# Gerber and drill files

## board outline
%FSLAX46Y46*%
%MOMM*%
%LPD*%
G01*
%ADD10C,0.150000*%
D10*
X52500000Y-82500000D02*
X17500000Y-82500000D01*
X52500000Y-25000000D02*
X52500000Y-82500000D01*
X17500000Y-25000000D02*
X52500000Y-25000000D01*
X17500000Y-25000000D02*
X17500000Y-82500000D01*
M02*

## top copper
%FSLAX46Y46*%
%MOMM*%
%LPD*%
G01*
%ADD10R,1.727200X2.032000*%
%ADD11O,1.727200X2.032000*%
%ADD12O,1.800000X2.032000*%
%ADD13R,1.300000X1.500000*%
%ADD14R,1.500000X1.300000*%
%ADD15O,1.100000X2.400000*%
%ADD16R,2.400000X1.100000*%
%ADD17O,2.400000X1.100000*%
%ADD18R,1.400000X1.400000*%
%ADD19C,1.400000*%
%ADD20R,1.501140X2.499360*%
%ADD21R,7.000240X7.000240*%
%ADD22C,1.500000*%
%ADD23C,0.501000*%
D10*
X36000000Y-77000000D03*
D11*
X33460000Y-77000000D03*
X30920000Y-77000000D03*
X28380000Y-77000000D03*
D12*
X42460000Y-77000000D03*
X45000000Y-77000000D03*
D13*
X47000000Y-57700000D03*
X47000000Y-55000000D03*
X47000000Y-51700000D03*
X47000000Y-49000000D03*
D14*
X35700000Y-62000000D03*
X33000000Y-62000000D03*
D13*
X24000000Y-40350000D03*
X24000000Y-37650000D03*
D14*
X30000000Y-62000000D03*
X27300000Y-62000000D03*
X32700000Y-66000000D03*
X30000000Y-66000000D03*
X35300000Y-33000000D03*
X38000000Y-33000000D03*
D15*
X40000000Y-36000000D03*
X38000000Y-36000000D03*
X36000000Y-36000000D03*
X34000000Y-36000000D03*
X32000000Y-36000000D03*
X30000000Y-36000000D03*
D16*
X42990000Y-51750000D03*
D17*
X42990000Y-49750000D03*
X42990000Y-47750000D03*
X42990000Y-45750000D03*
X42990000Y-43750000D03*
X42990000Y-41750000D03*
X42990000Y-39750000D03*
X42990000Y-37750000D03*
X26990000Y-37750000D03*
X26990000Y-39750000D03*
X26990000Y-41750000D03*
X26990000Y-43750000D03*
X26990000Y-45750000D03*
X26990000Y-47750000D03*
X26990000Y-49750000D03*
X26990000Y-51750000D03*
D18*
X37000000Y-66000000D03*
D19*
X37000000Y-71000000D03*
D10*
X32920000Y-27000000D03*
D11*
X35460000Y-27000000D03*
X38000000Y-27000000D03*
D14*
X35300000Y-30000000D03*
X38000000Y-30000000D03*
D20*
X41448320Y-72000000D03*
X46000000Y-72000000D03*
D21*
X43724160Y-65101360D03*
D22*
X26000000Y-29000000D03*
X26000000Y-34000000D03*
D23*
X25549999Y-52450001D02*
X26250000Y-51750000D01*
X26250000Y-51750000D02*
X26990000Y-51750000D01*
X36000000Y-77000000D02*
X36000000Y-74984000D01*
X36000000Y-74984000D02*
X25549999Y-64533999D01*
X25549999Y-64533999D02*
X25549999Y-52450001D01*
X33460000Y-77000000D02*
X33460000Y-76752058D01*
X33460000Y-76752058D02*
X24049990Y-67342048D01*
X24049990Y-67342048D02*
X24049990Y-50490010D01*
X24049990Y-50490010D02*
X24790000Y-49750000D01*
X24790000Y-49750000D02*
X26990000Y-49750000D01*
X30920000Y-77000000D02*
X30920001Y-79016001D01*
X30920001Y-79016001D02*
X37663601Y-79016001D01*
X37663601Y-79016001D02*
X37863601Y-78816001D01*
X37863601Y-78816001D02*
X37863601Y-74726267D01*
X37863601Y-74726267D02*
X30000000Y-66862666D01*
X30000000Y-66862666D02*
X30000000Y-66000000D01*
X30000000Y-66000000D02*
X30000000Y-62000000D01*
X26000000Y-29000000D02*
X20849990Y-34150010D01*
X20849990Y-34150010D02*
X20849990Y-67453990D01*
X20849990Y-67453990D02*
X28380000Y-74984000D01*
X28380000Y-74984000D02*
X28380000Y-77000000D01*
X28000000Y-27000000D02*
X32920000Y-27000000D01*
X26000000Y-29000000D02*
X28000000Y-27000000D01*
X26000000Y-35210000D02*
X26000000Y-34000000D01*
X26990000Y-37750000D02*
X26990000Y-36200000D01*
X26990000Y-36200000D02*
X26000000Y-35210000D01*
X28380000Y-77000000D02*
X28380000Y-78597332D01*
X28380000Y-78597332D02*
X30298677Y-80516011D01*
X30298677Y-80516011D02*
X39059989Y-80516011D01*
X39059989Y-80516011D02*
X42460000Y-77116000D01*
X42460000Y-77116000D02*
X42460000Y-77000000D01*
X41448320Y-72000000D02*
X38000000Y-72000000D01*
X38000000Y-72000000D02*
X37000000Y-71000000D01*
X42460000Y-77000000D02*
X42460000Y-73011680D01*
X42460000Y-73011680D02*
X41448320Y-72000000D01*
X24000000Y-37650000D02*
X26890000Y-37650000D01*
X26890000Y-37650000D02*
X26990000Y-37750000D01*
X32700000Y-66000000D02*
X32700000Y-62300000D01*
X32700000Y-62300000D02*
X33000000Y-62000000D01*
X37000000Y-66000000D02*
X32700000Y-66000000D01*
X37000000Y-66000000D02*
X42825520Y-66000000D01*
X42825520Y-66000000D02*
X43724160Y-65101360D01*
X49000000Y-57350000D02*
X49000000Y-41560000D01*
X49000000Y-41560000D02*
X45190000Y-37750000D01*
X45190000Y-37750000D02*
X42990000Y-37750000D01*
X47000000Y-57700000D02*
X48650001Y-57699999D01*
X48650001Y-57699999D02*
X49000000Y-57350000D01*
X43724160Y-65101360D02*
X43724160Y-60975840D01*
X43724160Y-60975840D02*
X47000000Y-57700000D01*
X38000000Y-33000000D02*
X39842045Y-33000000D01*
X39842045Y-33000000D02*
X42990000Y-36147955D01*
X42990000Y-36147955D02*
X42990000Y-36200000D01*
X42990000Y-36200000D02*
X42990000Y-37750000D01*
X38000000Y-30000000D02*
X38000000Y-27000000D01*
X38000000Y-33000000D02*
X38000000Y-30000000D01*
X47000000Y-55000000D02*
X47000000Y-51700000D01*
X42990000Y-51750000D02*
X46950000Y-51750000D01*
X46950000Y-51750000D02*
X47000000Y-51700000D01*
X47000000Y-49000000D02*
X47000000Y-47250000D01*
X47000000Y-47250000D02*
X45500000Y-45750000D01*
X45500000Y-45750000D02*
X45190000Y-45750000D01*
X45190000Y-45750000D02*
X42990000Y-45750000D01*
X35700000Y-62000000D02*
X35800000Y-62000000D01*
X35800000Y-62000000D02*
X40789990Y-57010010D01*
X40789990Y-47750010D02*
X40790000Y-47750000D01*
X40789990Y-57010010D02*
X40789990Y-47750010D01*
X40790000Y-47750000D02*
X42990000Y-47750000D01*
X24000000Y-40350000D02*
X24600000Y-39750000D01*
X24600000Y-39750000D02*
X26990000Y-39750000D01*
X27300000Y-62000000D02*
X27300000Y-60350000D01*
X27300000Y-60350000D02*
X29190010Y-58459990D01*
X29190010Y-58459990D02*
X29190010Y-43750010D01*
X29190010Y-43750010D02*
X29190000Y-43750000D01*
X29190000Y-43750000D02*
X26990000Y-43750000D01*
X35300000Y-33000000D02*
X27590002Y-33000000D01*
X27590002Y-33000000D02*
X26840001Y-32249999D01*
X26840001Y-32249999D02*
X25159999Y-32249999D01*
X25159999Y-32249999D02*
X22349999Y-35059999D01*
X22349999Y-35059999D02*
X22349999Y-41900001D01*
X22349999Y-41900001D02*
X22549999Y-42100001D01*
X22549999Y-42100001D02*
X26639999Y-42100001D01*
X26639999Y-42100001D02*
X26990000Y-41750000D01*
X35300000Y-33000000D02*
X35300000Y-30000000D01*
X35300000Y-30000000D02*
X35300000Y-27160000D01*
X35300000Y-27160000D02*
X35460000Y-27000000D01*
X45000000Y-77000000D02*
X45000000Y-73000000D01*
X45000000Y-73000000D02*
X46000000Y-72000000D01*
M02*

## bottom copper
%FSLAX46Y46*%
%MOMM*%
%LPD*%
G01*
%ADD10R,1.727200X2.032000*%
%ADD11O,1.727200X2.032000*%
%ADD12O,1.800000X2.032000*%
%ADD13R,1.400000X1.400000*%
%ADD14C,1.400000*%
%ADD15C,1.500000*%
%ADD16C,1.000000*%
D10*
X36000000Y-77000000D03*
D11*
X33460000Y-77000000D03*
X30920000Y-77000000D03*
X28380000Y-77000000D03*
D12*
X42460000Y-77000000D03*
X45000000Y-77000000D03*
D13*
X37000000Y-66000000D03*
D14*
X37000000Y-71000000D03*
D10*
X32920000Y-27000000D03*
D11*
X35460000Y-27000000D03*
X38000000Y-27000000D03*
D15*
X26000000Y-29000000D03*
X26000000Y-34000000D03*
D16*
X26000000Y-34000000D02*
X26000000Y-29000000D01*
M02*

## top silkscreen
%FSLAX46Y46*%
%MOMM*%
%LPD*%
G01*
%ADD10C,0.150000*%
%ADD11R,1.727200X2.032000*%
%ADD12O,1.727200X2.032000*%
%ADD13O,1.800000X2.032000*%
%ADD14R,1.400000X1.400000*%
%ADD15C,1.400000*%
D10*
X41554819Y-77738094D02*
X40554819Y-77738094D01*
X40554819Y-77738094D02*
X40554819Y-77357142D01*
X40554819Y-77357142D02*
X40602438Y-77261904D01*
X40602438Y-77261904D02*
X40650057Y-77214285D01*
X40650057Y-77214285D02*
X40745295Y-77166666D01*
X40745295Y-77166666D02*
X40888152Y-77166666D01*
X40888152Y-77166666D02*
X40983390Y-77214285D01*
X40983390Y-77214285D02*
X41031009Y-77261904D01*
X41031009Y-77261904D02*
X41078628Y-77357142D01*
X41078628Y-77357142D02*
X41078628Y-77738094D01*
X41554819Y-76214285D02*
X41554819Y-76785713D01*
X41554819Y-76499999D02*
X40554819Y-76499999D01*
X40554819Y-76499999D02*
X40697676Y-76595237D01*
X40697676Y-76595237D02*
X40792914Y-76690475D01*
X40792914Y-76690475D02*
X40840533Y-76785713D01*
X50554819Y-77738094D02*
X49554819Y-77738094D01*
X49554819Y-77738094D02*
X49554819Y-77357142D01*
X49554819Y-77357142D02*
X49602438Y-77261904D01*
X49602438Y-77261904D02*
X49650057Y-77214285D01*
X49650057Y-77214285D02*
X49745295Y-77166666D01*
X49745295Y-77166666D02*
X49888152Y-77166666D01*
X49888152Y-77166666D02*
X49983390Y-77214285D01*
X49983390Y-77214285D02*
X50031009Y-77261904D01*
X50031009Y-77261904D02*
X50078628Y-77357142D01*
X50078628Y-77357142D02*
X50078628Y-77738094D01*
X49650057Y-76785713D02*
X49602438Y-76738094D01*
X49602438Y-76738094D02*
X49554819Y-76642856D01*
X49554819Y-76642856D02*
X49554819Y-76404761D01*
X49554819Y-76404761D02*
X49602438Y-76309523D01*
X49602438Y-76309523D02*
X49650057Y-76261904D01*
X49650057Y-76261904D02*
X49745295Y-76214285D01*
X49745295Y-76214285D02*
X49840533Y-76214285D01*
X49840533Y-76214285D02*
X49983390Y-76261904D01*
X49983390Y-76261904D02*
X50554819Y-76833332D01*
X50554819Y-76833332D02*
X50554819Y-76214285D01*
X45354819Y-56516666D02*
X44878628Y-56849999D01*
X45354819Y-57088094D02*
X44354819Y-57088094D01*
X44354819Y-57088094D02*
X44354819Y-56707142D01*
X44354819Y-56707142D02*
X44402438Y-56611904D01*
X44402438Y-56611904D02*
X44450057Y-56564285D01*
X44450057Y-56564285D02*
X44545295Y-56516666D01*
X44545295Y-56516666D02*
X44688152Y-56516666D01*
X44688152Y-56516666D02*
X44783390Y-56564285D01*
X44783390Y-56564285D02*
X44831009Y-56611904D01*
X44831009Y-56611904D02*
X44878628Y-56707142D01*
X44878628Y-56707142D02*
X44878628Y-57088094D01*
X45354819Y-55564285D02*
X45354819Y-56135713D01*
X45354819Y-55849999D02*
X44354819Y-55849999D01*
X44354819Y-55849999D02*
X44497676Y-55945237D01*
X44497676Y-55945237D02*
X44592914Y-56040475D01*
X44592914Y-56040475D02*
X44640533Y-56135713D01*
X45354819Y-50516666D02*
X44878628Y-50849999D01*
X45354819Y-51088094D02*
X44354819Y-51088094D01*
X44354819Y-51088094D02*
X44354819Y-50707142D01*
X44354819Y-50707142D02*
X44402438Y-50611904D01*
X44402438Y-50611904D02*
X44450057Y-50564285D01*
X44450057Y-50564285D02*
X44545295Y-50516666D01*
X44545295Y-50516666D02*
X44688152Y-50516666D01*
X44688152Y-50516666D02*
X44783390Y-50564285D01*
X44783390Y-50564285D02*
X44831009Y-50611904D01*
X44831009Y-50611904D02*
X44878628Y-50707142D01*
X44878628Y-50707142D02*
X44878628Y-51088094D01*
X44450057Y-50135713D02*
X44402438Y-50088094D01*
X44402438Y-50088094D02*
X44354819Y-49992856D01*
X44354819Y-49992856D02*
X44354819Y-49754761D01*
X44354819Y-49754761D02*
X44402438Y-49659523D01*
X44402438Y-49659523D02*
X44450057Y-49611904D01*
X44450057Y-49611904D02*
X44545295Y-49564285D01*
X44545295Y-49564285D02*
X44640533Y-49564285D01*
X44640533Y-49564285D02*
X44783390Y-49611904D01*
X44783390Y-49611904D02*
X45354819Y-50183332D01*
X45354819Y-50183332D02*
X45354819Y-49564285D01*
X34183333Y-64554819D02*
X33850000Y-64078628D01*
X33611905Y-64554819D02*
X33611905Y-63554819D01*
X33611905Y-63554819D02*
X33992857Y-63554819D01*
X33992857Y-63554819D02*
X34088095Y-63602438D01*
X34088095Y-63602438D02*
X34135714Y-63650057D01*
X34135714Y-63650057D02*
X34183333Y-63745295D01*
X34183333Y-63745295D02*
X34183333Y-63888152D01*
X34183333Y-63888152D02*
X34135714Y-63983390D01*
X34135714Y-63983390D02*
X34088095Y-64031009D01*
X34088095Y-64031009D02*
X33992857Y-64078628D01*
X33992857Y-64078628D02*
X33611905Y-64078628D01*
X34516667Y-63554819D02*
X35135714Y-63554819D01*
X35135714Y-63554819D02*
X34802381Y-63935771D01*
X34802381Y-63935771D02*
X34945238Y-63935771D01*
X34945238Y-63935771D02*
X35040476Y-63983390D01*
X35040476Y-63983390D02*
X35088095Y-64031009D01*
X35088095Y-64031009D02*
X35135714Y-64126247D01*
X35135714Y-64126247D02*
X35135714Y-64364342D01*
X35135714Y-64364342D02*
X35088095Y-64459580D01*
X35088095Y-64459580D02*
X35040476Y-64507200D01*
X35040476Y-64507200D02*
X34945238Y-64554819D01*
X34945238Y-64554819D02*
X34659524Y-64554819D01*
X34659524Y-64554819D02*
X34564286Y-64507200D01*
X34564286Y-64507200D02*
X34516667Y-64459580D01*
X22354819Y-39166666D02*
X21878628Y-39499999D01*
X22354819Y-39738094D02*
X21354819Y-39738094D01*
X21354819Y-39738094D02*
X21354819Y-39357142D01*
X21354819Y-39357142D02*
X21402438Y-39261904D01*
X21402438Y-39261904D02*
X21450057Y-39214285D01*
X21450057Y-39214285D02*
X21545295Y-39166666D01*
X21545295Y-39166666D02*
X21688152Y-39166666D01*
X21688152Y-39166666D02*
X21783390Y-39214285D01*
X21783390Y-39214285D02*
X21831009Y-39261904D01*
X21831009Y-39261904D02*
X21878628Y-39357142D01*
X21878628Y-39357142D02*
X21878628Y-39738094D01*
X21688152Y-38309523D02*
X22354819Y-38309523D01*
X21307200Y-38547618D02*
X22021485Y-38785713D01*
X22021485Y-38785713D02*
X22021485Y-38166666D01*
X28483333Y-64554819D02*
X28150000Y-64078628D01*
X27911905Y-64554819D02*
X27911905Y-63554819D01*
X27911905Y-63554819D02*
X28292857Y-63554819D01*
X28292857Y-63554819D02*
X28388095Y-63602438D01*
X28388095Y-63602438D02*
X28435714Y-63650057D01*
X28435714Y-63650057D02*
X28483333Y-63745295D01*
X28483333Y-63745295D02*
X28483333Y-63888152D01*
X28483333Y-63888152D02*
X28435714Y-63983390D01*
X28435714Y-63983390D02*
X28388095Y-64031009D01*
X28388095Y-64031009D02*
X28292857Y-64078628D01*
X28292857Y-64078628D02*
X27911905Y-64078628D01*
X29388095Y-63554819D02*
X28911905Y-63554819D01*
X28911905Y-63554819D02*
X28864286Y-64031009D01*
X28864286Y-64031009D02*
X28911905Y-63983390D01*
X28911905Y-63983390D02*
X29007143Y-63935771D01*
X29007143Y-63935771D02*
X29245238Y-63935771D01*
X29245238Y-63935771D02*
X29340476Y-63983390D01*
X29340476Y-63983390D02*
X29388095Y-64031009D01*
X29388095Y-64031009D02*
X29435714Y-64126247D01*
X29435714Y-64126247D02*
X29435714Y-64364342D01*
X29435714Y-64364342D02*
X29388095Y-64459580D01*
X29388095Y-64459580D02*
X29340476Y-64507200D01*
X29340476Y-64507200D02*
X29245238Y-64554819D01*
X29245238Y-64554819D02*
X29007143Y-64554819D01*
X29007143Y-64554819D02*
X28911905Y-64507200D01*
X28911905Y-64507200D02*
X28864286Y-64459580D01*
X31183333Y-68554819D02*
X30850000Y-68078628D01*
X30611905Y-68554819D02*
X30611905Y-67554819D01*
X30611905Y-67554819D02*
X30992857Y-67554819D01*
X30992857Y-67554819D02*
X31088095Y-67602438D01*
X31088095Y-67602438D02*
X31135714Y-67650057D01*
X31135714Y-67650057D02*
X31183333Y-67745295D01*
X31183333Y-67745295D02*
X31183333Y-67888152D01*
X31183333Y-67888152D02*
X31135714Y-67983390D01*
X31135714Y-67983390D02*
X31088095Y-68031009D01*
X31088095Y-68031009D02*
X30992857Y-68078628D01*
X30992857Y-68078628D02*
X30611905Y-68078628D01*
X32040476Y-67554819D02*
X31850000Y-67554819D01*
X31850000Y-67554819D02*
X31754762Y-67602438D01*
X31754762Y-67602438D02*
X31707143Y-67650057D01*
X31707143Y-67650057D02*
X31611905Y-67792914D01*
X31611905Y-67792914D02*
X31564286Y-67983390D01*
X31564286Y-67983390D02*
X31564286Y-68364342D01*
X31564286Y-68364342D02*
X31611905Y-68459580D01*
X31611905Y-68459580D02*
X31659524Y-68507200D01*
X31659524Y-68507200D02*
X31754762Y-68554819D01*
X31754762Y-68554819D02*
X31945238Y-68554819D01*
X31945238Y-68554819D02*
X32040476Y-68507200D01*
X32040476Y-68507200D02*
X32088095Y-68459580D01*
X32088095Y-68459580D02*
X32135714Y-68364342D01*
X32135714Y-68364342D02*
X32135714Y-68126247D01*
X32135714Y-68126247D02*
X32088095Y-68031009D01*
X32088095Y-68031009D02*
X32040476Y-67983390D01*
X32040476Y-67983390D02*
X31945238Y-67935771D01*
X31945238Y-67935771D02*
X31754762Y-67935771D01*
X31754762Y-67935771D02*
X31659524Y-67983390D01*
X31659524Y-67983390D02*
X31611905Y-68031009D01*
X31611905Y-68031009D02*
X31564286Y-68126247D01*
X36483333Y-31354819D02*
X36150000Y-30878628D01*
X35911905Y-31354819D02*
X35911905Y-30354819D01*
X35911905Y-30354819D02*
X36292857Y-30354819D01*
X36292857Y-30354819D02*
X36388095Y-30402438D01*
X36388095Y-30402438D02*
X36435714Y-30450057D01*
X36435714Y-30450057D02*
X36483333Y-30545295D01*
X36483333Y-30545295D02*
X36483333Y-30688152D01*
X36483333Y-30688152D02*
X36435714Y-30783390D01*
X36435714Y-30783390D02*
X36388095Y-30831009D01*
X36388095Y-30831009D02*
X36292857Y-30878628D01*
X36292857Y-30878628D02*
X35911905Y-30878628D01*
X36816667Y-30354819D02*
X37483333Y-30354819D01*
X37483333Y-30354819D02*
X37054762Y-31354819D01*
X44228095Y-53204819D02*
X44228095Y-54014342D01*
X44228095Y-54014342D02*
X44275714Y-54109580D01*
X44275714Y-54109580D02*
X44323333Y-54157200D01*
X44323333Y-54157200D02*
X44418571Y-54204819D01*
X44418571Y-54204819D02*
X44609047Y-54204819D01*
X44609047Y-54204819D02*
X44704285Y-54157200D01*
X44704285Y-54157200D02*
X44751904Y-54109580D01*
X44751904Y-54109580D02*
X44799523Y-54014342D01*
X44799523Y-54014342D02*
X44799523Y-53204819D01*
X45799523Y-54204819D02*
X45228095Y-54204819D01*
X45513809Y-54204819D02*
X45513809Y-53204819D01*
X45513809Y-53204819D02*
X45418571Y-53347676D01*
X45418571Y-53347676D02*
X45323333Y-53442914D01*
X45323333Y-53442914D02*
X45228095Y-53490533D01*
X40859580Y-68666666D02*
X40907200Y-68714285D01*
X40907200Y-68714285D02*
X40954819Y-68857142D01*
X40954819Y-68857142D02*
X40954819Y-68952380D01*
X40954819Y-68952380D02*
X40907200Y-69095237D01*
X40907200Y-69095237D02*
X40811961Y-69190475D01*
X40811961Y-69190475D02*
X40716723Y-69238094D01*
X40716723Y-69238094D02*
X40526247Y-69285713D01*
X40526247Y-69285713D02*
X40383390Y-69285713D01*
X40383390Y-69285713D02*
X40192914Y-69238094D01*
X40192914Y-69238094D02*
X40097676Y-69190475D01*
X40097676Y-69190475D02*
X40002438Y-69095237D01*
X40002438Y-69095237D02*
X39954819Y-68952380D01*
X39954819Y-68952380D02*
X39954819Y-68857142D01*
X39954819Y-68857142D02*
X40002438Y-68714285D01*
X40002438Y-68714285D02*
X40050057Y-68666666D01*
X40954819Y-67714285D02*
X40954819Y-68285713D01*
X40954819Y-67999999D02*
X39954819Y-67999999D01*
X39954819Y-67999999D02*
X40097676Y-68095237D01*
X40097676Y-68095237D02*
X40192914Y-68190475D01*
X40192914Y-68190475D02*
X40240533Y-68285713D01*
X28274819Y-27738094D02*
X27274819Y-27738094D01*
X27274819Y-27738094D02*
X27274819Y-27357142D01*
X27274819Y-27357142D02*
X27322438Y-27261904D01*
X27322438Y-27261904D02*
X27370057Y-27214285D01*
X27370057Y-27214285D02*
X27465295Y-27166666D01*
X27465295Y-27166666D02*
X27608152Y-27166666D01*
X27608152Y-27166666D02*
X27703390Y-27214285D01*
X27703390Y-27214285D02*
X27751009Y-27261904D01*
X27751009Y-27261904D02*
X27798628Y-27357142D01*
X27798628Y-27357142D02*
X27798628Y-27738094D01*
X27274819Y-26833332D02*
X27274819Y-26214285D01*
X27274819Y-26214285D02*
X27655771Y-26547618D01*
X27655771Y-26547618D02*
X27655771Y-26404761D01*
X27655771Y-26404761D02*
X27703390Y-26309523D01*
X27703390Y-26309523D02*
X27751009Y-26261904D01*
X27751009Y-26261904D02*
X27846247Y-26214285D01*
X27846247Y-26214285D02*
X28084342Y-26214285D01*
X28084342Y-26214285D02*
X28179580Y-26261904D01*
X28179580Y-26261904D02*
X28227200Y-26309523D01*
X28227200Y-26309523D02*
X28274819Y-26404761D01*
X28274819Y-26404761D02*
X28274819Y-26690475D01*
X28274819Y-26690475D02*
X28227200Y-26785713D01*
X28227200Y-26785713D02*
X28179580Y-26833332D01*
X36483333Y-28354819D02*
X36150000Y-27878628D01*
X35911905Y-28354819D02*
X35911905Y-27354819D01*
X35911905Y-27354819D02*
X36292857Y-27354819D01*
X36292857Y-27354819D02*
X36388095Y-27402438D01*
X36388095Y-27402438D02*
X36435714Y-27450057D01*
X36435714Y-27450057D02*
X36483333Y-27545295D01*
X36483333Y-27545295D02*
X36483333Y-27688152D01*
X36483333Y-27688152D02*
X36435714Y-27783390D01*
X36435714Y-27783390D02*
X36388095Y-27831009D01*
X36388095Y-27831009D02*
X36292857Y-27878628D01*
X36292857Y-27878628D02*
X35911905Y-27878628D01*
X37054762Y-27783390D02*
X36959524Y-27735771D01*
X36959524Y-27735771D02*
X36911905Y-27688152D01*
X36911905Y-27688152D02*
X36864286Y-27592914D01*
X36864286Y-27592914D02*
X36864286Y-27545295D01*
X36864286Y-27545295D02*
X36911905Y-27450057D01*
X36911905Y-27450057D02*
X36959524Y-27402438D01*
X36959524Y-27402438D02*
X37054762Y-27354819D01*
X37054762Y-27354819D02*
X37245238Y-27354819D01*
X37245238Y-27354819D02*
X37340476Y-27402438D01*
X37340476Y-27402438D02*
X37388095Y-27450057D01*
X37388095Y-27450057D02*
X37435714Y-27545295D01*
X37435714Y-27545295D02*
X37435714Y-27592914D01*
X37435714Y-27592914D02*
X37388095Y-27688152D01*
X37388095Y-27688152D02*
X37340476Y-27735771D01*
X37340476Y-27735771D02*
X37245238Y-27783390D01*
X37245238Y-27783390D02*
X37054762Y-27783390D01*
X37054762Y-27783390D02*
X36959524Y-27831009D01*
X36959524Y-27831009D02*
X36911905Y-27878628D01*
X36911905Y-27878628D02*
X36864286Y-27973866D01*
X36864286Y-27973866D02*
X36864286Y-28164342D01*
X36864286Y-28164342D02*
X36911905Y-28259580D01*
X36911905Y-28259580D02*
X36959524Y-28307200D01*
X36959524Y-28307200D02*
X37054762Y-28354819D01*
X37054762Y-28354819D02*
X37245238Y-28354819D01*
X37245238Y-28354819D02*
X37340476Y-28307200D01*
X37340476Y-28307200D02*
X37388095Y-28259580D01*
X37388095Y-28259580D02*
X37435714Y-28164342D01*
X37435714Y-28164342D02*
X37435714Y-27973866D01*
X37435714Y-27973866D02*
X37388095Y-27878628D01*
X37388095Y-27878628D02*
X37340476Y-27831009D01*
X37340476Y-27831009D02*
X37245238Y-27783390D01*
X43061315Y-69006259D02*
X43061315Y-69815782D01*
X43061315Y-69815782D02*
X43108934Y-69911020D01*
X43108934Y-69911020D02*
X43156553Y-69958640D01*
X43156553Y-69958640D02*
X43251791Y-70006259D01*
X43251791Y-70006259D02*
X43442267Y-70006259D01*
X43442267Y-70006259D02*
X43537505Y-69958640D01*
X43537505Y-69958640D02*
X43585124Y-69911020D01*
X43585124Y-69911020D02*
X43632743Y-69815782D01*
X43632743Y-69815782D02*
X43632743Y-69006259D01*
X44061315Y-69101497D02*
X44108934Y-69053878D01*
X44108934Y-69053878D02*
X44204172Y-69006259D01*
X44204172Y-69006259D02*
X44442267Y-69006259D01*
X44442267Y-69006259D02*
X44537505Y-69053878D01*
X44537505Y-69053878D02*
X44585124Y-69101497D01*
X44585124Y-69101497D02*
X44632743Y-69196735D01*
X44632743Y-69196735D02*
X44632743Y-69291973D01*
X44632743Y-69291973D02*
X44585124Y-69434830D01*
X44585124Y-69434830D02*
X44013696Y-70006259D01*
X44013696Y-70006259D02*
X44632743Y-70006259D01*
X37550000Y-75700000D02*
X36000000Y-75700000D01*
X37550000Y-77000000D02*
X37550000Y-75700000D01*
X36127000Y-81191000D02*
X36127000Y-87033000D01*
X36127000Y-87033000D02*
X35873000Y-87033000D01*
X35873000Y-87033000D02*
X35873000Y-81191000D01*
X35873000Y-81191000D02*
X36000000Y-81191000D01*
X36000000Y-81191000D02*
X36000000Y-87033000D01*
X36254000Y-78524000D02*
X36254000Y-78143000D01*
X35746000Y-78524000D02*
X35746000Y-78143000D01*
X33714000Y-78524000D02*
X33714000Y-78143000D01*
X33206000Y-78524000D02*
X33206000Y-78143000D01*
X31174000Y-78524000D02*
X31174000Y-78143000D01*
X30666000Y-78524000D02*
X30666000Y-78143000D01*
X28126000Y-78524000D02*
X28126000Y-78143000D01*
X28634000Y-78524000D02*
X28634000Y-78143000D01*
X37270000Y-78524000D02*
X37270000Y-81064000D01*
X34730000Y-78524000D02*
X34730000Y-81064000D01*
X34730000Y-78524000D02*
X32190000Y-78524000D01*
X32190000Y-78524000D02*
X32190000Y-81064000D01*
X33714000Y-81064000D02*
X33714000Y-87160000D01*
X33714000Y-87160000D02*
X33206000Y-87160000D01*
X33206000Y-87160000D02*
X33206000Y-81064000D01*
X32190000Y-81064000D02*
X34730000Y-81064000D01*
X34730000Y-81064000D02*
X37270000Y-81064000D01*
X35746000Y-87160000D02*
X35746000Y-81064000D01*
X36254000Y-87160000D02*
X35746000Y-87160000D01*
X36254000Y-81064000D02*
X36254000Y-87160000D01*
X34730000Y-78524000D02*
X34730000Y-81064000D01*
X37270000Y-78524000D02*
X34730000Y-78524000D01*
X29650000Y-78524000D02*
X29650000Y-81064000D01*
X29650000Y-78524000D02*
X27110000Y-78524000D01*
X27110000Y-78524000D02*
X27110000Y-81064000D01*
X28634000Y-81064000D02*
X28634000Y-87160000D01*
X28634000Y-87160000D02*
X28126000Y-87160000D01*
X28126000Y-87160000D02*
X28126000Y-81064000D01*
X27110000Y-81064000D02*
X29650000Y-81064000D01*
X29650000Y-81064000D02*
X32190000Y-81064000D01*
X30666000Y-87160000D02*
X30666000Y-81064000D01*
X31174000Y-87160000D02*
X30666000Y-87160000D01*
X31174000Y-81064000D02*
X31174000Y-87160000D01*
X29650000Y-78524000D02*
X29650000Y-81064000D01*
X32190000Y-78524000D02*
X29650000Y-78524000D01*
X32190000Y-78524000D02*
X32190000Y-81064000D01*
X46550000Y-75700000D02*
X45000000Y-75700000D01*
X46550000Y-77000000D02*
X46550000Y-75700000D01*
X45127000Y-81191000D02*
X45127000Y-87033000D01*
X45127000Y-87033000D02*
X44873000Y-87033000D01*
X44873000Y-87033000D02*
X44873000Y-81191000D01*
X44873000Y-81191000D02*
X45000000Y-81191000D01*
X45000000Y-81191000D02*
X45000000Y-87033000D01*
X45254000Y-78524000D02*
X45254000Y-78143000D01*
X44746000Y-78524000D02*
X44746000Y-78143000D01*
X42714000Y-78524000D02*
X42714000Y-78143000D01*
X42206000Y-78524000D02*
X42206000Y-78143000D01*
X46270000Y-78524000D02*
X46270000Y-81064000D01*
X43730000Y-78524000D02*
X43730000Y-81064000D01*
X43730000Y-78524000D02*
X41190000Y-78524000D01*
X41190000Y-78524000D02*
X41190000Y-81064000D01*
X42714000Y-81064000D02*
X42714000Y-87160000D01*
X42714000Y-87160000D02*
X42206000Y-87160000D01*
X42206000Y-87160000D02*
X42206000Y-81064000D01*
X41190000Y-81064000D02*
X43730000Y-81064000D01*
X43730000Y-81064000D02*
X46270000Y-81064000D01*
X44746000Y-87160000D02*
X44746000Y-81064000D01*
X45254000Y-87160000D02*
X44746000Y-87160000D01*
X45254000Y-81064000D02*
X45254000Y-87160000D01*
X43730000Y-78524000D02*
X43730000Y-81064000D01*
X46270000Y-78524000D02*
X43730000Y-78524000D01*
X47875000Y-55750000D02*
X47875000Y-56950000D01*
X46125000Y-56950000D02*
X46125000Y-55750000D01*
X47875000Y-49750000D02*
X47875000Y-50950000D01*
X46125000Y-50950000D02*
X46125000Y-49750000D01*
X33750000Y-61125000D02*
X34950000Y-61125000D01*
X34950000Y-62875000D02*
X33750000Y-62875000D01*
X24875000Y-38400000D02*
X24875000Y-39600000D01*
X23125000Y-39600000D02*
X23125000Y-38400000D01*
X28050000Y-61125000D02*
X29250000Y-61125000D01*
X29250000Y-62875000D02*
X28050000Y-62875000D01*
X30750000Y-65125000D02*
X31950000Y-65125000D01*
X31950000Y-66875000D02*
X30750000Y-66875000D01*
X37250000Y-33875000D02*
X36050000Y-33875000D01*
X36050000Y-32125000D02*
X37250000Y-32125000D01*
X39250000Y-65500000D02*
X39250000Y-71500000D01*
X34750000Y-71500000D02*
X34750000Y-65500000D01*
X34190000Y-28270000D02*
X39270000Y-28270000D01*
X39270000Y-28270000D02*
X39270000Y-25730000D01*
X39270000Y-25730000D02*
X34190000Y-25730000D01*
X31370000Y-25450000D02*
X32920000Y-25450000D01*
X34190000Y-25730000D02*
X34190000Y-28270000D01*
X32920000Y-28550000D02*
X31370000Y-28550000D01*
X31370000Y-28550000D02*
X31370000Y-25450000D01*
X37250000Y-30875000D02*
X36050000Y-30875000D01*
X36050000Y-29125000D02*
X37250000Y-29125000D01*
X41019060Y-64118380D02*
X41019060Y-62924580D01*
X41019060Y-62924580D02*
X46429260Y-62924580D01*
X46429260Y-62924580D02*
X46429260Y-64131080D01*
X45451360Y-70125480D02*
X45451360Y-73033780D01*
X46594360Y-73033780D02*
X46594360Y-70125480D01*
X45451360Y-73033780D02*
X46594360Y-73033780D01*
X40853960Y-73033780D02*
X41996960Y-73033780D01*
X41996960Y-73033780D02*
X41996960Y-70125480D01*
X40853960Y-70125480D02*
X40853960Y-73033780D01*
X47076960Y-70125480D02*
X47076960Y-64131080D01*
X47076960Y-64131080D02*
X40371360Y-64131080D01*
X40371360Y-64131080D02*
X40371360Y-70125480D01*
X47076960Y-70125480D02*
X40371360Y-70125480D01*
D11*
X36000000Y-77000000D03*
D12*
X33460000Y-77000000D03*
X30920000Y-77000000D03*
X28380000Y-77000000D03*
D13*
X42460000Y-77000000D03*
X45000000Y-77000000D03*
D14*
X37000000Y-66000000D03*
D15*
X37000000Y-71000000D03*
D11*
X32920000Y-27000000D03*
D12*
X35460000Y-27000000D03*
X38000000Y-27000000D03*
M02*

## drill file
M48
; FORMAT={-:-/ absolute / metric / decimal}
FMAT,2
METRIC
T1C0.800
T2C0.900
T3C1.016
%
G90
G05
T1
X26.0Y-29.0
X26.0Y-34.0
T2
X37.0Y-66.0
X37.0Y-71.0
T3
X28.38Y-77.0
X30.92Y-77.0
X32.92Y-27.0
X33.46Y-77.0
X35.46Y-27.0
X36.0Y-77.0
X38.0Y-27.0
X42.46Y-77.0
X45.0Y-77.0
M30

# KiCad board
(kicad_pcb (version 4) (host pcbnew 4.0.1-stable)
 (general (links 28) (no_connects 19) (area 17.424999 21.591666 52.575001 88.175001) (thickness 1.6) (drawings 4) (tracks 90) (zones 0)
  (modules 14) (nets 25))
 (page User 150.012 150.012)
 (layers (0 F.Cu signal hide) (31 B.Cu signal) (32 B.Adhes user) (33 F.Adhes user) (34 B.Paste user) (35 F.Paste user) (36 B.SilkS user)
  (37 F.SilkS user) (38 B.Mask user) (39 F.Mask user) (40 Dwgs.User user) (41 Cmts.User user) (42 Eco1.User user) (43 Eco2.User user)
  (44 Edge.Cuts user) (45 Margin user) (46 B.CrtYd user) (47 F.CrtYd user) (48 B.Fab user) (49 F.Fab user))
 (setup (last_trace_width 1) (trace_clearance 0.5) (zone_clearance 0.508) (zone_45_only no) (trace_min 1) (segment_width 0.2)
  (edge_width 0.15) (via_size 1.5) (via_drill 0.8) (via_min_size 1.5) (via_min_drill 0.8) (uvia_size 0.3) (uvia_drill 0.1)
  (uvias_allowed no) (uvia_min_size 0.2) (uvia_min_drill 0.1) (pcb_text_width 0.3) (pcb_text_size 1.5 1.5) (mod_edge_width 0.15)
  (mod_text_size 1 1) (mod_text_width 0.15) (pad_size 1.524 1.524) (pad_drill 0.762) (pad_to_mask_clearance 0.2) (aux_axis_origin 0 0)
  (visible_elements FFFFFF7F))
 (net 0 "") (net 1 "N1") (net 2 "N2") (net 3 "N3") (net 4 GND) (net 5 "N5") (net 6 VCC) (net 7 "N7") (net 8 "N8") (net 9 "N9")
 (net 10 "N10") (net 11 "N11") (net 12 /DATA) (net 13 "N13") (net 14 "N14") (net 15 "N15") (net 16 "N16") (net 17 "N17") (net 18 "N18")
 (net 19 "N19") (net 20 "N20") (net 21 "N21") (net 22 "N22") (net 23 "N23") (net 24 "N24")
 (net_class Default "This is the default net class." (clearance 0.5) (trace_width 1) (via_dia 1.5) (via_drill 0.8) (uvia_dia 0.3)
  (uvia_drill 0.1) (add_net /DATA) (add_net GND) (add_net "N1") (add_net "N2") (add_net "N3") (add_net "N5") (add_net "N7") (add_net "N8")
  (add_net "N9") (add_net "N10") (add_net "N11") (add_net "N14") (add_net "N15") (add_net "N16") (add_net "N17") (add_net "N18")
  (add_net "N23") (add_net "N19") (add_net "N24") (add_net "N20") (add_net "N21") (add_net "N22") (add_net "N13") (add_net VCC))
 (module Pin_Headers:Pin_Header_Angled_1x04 (layer F.Cu) (at 36 77 270)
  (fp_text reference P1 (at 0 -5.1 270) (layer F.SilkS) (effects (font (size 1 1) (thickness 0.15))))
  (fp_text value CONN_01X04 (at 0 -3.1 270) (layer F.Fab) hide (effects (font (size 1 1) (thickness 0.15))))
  (fp_line (start -1.3 -1.55) (end -1.3 0) (layer F.SilkS) (width 0.15))
  (fp_line (start 0 -1.55) (end -1.3 -1.55) (layer F.SilkS) (width 0.15))
  (fp_line (start 4.191 -0.127) (end 10.033 -0.127) (layer F.SilkS) (width 0.15))
  (fp_line (start 10.033 -0.127) (end 10.033 0.127) (layer F.SilkS) (width 0.15))
  (fp_line (start 10.033 0.127) (end 4.191 0.127) (layer F.SilkS) (width 0.15))
  (fp_line (start 4.191 0.127) (end 4.191 0) (layer F.SilkS) (width 0.15))
  (fp_line (start 4.191 0) (end 10.033 0) (layer F.SilkS) (width 0.15))
  (fp_line (start 1.524 -0.254) (end 1.143 -0.254) (layer F.SilkS) (width 0.15))
  (fp_line (start 1.524 0.254) (end 1.143 0.254) (layer F.SilkS) (width 0.15))
  (fp_line (start 1.524 2.286) (end 1.143 2.286) (layer F.SilkS) (width 0.15))
  (fp_line (start 1.524 2.794) (end 1.143 2.794) (layer F.SilkS) (width 0.15))
  (fp_line (start 1.524 4.826) (end 1.143 4.826) (layer F.SilkS) (width 0.15))
  (fp_line (start 1.524 5.334) (end 1.143 5.334) (layer F.SilkS) (width 0.15))
  (fp_line (start 1.524 7.874) (end 1.143 7.874) (layer F.SilkS) (width 0.15))
  (fp_line (start 1.524 7.366) (end 1.143 7.366) (layer F.SilkS) (width 0.15))
  (fp_line (start 1.524 -1.27) (end 4.064 -1.27) (layer F.SilkS) (width 0.15))
  (fp_line (start 1.524 1.27) (end 4.064 1.27) (layer F.SilkS) (width 0.15))
  (fp_line (start 1.524 1.27) (end 1.524 3.81) (layer F.SilkS) (width 0.15))
  (fp_line (start 1.524 3.81) (end 4.064 3.81) (layer F.SilkS) (width 0.15))
  (fp_line (start 4.064 2.286) (end 10.16 2.286) (layer F.SilkS) (width 0.15))
  (fp_line (start 10.16 2.286) (end 10.16 2.794) (layer F.SilkS) (width 0.15))
  (fp_line (start 10.16 2.794) (end 4.064 2.794) (layer F.SilkS) (width 0.15))
  (fp_line (start 4.064 3.81) (end 4.064 1.27) (layer F.SilkS) (width 0.15))
  (fp_line (start 4.064 1.27) (end 4.064 -1.27) (layer F.SilkS) (width 0.15))
  (fp_line (start 10.16 0.254) (end 4.064 0.254) (layer F.SilkS) (width 0.15))
  (fp_line (start 10.16 -0.254) (end 10.16 0.254) (layer F.SilkS) (width 0.15))
  (fp_line (start 4.064 -0.254) (end 10.16 -0.254) (layer F.SilkS) (width 0.15))
  (fp_line (start 1.524 1.27) (end 4.064 1.27) (layer F.SilkS) (width 0.15))
  (fp_line (start 1.524 -1.27) (end 1.524 1.27) (layer F.SilkS) (width 0.15))
  (fp_line (start 1.524 6.35) (end 4.064 6.35) (layer F.SilkS) (width 0.15))
  (fp_line (start 1.524 6.35) (end 1.524 8.89) (layer F.SilkS) (width 0.15))
  (fp_line (start 1.524 8.89) (end 4.064 8.89) (layer F.SilkS) (width 0.15))
  (fp_line (start 4.064 7.366) (end 10.16 7.366) (layer F.SilkS) (width 0.15))
  (fp_line (start 10.16 7.366) (end 10.16 7.874) (layer F.SilkS) (width 0.15))
  (fp_line (start 10.16 7.874) (end 4.064 7.874) (layer F.SilkS) (width 0.15))
  (fp_line (start 4.064 8.89) (end 4.064 6.35) (layer F.SilkS) (width 0.15))
  (fp_line (start 4.064 6.35) (end 4.064 3.81) (layer F.SilkS) (width 0.15))
  (fp_line (start 10.16 5.334) (end 4.064 5.334) (layer F.SilkS) (width 0.15))
  (fp_line (start 10.16 4.826) (end 10.16 5.334) (layer F.SilkS) (width 0.15))
  (fp_line (start 4.064 4.826) (end 10.16 4.826) (layer F.SilkS) (width 0.15))
  (fp_line (start 1.524 6.35) (end 4.064 6.35) (layer F.SilkS) (width 0.15))
  (fp_line (start 1.524 3.81) (end 1.524 6.35) (layer F.SilkS) (width 0.15))
  (fp_line (start 1.524 3.81) (end 4.064 3.81) (layer F.SilkS) (width 0.15))
  (pad 1 thru_hole rect (at 0 0 270) (size 2.032 1.7272) (drill 1.016) (layers *.Cu *.Mask F.SilkS) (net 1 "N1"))
  (pad 2 thru_hole oval (at 0 2.54 270) (size 2.032 1.7272) (drill 1.016) (layers *.Cu *.Mask F.SilkS) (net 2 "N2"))
  (pad 3 thru_hole oval (at 0 5.08 270) (size 2.032 1.7272) (drill 1.016) (layers *.Cu *.Mask F.SilkS) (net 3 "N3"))
  (pad 4 thru_hole oval (at 0 7.62 270) (size 2.032 1.7272) (drill 1.016) (layers *.Cu *.Mask F.SilkS) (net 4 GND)))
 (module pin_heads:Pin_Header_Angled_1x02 (layer F.Cu) (at 45 77 270)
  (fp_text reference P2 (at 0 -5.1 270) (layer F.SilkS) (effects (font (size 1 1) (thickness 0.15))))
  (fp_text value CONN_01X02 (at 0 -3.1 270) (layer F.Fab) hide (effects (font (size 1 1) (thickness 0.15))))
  (fp_line (start -1.3 -1.55) (end -1.3 0) (layer F.SilkS) (width 0.15))
  (fp_line (start 0 -1.55) (end -1.3 -1.55) (layer F.SilkS) (width 0.15))
  (fp_line (start 4.191 -0.127) (end 10.033 -0.127) (layer F.SilkS) (width 0.15))
  (fp_line (start 10.033 -0.127) (end 10.033 0.127) (layer F.SilkS) (width 0.15))
  (fp_line (start 10.033 0.127) (end 4.191 0.127) (layer F.SilkS) (width 0.15))
  (fp_line (start 4.191 0.127) (end 4.191 0) (layer F.SilkS) (width 0.15))
  (fp_line (start 4.191 0) (end 10.033 0) (layer F.SilkS) (width 0.15))
  (fp_line (start 1.524 -0.254) (end 1.143 -0.254) (layer F.SilkS) (width 0.15))
  (fp_line (start 1.524 0.254) (end 1.143 0.254) (layer F.SilkS) (width 0.15))
  (fp_line (start 1.524 2.286) (end 1.143 2.286) (layer F.SilkS) (width 0.15))
  (fp_line (start 1.524 2.794) (end 1.143 2.794) (layer F.SilkS) (width 0.15))
  (fp_line (start 1.524 -1.27) (end 4.064 -1.27) (layer F.SilkS) (width 0.15))
  (fp_line (start 1.524 1.27) (end 4.064 1.27) (layer F.SilkS) (width 0.15))
  (fp_line (start 1.524 1.27) (end 1.524 3.81) (layer F.SilkS) (width 0.15))
  (fp_line (start 1.524 3.81) (end 4.064 3.81) (layer F.SilkS) (width 0.15))
  (fp_line (start 4.064 2.286) (end 10.16 2.286) (layer F.SilkS) (width 0.15))
  (fp_line (start 10.16 2.286) (end 10.16 2.794) (layer F.SilkS) (width 0.15))
  (fp_line (start 10.16 2.794) (end 4.064 2.794) (layer F.SilkS) (width 0.15))
  (fp_line (start 4.064 3.81) (end 4.064 1.27) (layer F.SilkS) (width 0.15))
  (fp_line (start 4.064 1.27) (end 4.064 -1.27) (layer F.SilkS) (width 0.15))
  (fp_line (start 10.16 0.254) (end 4.064 0.254) (layer F.SilkS) (width 0.15))
  (fp_line (start 10.16 -0.254) (end 10.16 0.254) (layer F.SilkS) (width 0.15))
  (fp_line (start 4.064 -0.254) (end 10.16 -0.254) (layer F.SilkS) (width 0.15))
  (fp_line (start 1.524 1.27) (end 4.064 1.27) (layer F.SilkS) (width 0.15))
  (fp_line (start 1.524 -1.27) (end 1.524 1.27) (layer F.SilkS) (width 0.15))
  (pad 2 thru_hole oval (at 0 2.54 270) (size 2.032 1.8) (drill 1.016) (layers *.Cu *.Mask F.SilkS) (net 4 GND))
  (pad 1 thru_hole oval (at 0 0 270) (size 2.032 1.8) (drill 1.016) (layers *.Cu *.Mask F.SilkS) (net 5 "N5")))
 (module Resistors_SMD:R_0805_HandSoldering (layer F.Cu) (at 47 56.35 90)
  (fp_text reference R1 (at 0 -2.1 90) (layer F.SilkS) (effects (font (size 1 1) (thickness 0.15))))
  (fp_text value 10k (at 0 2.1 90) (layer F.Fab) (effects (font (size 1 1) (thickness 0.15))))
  (fp_line (start 0.6 0.875) (end -0.6 0.875) (layer F.SilkS) (width 0.15))
  (fp_line (start -0.6 -0.875) (end 0.6 -0.875) (layer F.SilkS) (width 0.15))
  (pad 1 smd rect (at -1.35 0 90) (size 1.5 1.3) (layers F.Cu F.Paste F.Mask) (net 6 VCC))
  (pad 2 smd rect (at 1.35 0 90) (size 1.5 1.3) (layers F.Cu F.Paste F.Mask) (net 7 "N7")))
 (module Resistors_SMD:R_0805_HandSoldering (layer F.Cu) (at 47 50.35 90)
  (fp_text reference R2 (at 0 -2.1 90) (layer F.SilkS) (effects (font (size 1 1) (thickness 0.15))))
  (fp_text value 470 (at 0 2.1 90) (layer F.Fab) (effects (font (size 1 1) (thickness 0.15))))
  (fp_line (start 0.6 0.875) (end -0.6 0.875) (layer F.SilkS) (width 0.15))
  (fp_line (start -0.6 -0.875) (end 0.6 -0.875) (layer F.SilkS) (width 0.15))
  (pad 1 smd rect (at -1.35 0 90) (size 1.5 1.3) (layers F.Cu F.Paste F.Mask) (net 7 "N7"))
  (pad 2 smd rect (at 1.35 0 90) (size 1.5 1.3) (layers F.Cu F.Paste F.Mask) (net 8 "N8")))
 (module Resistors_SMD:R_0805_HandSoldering (layer F.Cu) (at 34.35 62 180)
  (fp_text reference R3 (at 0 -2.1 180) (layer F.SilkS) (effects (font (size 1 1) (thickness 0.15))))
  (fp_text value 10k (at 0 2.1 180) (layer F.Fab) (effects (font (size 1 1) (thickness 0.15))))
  (fp_line (start 0.6 0.875) (end -0.6 0.875) (layer F.SilkS) (width 0.15))
  (fp_line (start -0.6 -0.875) (end 0.6 -0.875) (layer F.SilkS) (width 0.15))
  (pad 1 smd rect (at -1.35 0 180) (size 1.5 1.3) (layers F.Cu F.Paste F.Mask) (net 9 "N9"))
  (pad 2 smd rect (at 1.35 0 180) (size 1.5 1.3) (layers F.Cu F.Paste F.Mask) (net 6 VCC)))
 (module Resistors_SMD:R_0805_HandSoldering (layer F.Cu) (at 24 39 90)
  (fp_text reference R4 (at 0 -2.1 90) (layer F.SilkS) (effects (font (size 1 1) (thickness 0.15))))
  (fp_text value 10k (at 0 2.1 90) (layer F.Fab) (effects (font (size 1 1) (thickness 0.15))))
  (fp_line (start 0.6 0.875) (end -0.6 0.875) (layer F.SilkS) (width 0.15))
  (fp_line (start -0.6 -0.875) (end 0.6 -0.875) (layer F.SilkS) (width 0.15))
  (pad 1 smd rect (at -1.35 0 90) (size 1.5 1.3) (layers F.Cu F.Paste F.Mask) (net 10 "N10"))
  (pad 2 smd rect (at 1.35 0 90) (size 1.5 1.3) (layers F.Cu F.Paste F.Mask) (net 4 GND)))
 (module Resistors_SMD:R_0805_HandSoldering (layer F.Cu) (at 28.65 62 180)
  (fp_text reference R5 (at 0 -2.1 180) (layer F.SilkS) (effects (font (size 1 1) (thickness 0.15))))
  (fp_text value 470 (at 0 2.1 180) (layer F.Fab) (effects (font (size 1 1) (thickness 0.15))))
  (fp_line (start 0.6 0.875) (end -0.6 0.875) (layer F.SilkS) (width 0.15))
  (fp_line (start -0.6 -0.875) (end 0.6 -0.875) (layer F.SilkS) (width 0.15))
  (pad 1 smd rect (at -1.35 0 180) (size 1.5 1.3) (layers F.Cu F.Paste F.Mask) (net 3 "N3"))
  (pad 2 smd rect (at 1.35 0 180) (size 1.5 1.3) (layers F.Cu F.Paste F.Mask) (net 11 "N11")))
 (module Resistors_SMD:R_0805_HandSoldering (layer F.Cu) (at 31.35 66 180)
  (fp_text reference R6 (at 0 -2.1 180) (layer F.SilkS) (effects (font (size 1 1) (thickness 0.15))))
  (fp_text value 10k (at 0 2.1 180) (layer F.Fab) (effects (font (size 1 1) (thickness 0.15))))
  (fp_line (start 0.6 0.875) (end -0.6 0.875) (layer F.SilkS) (width 0.15))
  (fp_line (start -0.6 -0.875) (end 0.6 -0.875) (layer F.SilkS) (width 0.15))
  (pad 1 smd rect (at -1.35 0 180) (size 1.5 1.3) (layers F.Cu F.Paste F.Mask) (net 6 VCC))
  (pad 2 smd rect (at 1.35 0 180) (size 1.5 1.3) (layers F.Cu F.Paste F.Mask) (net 3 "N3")))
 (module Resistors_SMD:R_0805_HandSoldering (layer F.Cu) (at 36.65 33)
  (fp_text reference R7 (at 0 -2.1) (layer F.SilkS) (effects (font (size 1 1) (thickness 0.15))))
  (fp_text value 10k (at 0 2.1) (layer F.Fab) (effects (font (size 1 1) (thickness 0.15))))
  (fp_line (start 0.6 0.875) (end -0.6 0.875) (layer F.SilkS) (width 0.15))
  (fp_line (start -0.6 -0.875) (end 0.6 -0.875) (layer F.SilkS) (width 0.15))
  (pad 1 smd rect (at -1.35 0) (size 1.5 1.3) (layers F.Cu F.Paste F.Mask) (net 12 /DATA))
  (pad 2 smd rect (at 1.35 0) (size 1.5 1.3) (layers F.Cu F.Paste F.Mask) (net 6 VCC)))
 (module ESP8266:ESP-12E (layer F.Cu) (at 42.99 51.75 180)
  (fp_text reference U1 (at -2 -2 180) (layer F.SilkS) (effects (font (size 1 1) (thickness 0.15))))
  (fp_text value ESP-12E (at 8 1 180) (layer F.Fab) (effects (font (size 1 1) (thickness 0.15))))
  (pad 9 smd oval (at 2.99 15.75 270) (size 2.4 1.1) (layers F.Cu F.Paste F.Mask) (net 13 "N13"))
  (pad 10 smd oval (at 4.99 15.75 270) (size 2.4 1.1) (layers F.Cu F.Paste F.Mask) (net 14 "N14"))
  (pad 11 smd oval (at 6.99 15.75 270) (size 2.4 1.1) (layers F.Cu F.Paste F.Mask) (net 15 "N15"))
  (pad 12 smd oval (at 8.99 15.75 270) (size 2.4 1.1) (layers F.Cu F.Paste F.Mask) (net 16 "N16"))
  (pad 13 smd oval (at 10.99 15.75 270) (size 2.4 1.1) (layers F.Cu F.Paste F.Mask) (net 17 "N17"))
  (pad 14 smd oval (at 12.99 15.75 270) (size 2.4 1.1) (layers F.Cu F.Paste F.Mask) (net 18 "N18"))
  (pad 1 smd rect (at 0 0 180) (size 2.4 1.1) (layers F.Cu F.Paste F.Mask) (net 7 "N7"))
  (pad 2 smd oval (at 0 2 180) (size 2.4 1.1) (layers F.Cu F.Paste F.Mask) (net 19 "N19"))
  (pad 3 smd oval (at 0 4 180) (size 2.4 1.1) (layers F.Cu F.Paste F.Mask) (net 9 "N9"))
  (pad 4 smd oval (at 0 6 180) (size 2.4 1.1) (layers F.Cu F.Paste F.Mask) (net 8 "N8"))
  (pad 5 smd oval (at 0 8 180) (size 2.4 1.1) (layers F.Cu F.Paste F.Mask) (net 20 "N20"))
  (pad 6 smd oval (at 0 10 180) (size 2.4 1.1) (layers F.Cu F.Paste F.Mask) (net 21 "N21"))
  (pad 7 smd oval (at 0 12 180) (size 2.4 1.1) (layers F.Cu F.Paste F.Mask) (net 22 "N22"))
  (pad 8 smd oval (at 0 14 180) (size 2.4 1.1) (layers F.Cu F.Paste F.Mask) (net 6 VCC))
  (pad 15 smd oval (at 16 14 180) (size 2.4 1.1) (layers F.Cu F.Paste F.Mask) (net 4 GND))
  (pad 16 smd oval (at 16 12 180) (size 2.4 1.1) (layers F.Cu F.Paste F.Mask) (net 10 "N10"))
  (pad 17 smd oval (at 16 10 180) (size 2.4 1.1) (layers F.Cu F.Paste F.Mask) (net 12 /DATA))
  (pad 18 smd oval (at 16 8 180) (size 2.4 1.1) (layers F.Cu F.Paste F.Mask) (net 11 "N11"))
  (pad 19 smd oval (at 16 6 180) (size 2.4 1.1) (layers F.Cu F.Paste F.Mask) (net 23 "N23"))
  (pad 20 smd oval (at 16 4 180) (size 2.4 1.1) (layers F.Cu F.Paste F.Mask) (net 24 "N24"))
  (pad 21 smd oval (at 16 2 180) (size 2.4 1.1) (layers F.Cu F.Paste F.Mask) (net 2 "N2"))
  (pad 22 smd oval (at 16 0 180) (size 2.4 1.1) (layers F.Cu F.Paste F.Mask) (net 1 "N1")))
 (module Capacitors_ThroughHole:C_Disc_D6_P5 (layer F.Cu) (at 37 66 270)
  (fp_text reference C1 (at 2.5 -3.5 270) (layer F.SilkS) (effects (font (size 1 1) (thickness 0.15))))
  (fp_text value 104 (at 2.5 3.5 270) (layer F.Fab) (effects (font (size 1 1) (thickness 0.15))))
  (fp_line (start -0.5 -2.25) (end 5.5 -2.25) (layer F.SilkS) (width 0.15))
  (fp_line (start 5.5 2.25) (end -0.5 2.25) (layer F.SilkS) (width 0.15))
  (pad 1 thru_hole rect (at 0 0 270) (size 1.4 1.4) (drill 0.9) (layers *.Cu *.Mask F.SilkS) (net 6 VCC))
  (pad 2 thru_hole circle (at 5 0 270) (size 1.4 1.4) (drill 0.9) (layers *.Cu *.Mask F.SilkS) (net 4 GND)))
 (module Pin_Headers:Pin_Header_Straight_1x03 (layer F.Cu) (at 32.92 27 90)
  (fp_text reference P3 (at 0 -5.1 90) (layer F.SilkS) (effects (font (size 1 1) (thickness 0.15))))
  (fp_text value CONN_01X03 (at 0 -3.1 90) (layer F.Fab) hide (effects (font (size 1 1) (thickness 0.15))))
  (fp_line (start -1.27 1.27) (end -1.27 6.35) (layer F.SilkS) (width 0.15))
  (fp_line (start -1.27 6.35) (end 1.27 6.35) (layer F.SilkS) (width 0.15))
  (fp_line (start 1.27 6.35) (end 1.27 1.27) (layer F.SilkS) (width 0.15))
  (fp_line (start 1.55 -1.55) (end 1.55 0) (layer F.SilkS) (width 0.15))
  (fp_line (start 1.27 1.27) (end -1.27 1.27) (layer F.SilkS) (width 0.15))
  (fp_line (start -1.55 0) (end -1.55 -1.55) (layer F.SilkS) (width 0.15))
  (fp_line (start -1.55 -1.55) (end 1.55 -1.55) (layer F.SilkS) (width 0.15))
  (pad 1 thru_hole rect (at 0 0 90) (size 2.032 1.7272) (drill 1.016) (layers *.Cu *.Mask F.SilkS) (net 4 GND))
  (pad 2 thru_hole oval (at 0 2.54 90) (size 2.032 1.7272) (drill 1.016) (layers *.Cu *.Mask F.SilkS) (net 12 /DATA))
  (pad 3 thru_hole oval (at 0 5.08 90) (size 2.032 1.7272) (drill 1.016) (layers *.Cu *.Mask F.SilkS) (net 6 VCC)))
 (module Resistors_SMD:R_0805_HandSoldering (layer F.Cu) (at 36.65 30)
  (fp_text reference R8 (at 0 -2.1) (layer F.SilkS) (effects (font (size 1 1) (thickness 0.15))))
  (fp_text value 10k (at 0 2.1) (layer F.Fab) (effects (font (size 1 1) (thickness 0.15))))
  (fp_line (start 0.6 0.875) (end -0.6 0.875) (layer F.SilkS) (width 0.15))
  (fp_line (start -0.6 -0.875) (end 0.6 -0.875) (layer F.SilkS) (width 0.15))
  (pad 1 smd rect (at -1.35 0) (size 1.5 1.3) (layers F.Cu F.Paste F.Mask) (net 12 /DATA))
  (pad 2 smd rect (at 1.35 0) (size 1.5 1.3) (layers F.Cu F.Paste F.Mask) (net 6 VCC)))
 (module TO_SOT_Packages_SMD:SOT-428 (layer F.Cu) (at 43.72416 68.55068)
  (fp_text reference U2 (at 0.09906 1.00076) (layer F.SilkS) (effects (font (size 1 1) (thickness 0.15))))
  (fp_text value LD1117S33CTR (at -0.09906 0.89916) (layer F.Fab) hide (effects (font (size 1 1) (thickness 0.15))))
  (fp_line (start -2.7051 -4.4323) (end -2.7051 -5.6261) (layer F.SilkS) (width 0.15))
  (fp_line (start -2.7051 -5.6261) (end 2.7051 -5.6261) (layer F.SilkS) (width 0.15))
  (fp_line (start 2.7051 -5.6261) (end 2.7051 -4.4196) (layer F.SilkS) (width 0.15))
  (fp_line (start 1.7272 1.5748) (end 1.7272 4.4831) (layer F.SilkS) (width 0.15))
  (fp_line (start 2.8702 4.4831) (end 2.8702 1.5748) (layer F.SilkS) (width 0.15))
  (fp_line (start 1.7272 4.4831) (end 2.8702 4.4831) (layer F.SilkS) (width 0.15))
  (fp_line (start -2.8702 4.4831) (end -1.7272 4.4831) (layer F.SilkS) (width 0.15))
  (fp_line (start -1.7272 4.4831) (end -1.7272 1.5748) (layer F.SilkS) (width 0.15))
  (fp_line (start -2.8702 1.5748) (end -2.8702 4.4831) (layer F.SilkS) (width 0.15))
  (fp_line (start 3.3528 1.5748) (end 3.3528 -4.4196) (layer F.SilkS) (width 0.15))
  (fp_line (start 3.3528 -4.4196) (end -3.3528 -4.4196) (layer F.SilkS) (width 0.15))
  (fp_line (start -3.3528 -4.4196) (end -3.3528 1.5748) (layer F.SilkS) (width 0.15))
  (fp_line (start 3.3528 1.5748) (end -3.3528 1.5748) (layer F.SilkS) (width 0.15))
  (pad 1 smd rect (at -2.27584 3.44932) (size 1.50114 2.49936) (layers F.Cu F.Paste F.Mask) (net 4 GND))
  (pad 3 smd rect (at 2.27584 3.44932) (size 1.50114 2.49936) (layers F.Cu F.Paste F.Mask) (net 5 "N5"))
  (pad 2 smd rect (at 0 -3.44932) (size 7.00024 7.00024) (layers F.Cu F.Paste F.Mask) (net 6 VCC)))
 (gr_line (start 52.5 82.5) (end 17.5 82.5) (layer Edge.Cuts) (width 0.15))
 (gr_line (start 52.5 25) (end 52.5 82.5) (layer Edge.Cuts) (width 0.15))
 (gr_line (start 17.5 25) (end 52.5 25) (layer Edge.Cuts) (width 0.15))
 (gr_line (start 17.5 25) (end 17.5 82.5) (layer Edge.Cuts) (width 0.15))
 (segment (start 25.549999 52.450001) (end 26.25 51.75) (width 0.501) (layer F.Cu) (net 1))
 (segment (start 26.25 51.75) (end 26.99 51.75) (width 0.501) (layer F.Cu) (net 1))
 (segment (start 36 77) (end 36 74.984) (width 0.501) (layer F.Cu) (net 1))
 (segment (start 36 74.984) (end 25.549999 64.533999) (width 0.501) (layer F.Cu) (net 1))
 (segment (start 25.549999 64.533999) (end 25.549999 52.450001) (width 0.501) (layer F.Cu) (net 1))
 (segment (start 33.46 77) (end 33.46 76.752058) (width 0.501) (layer F.Cu) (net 2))
 (segment (start 33.46 76.752058) (end 24.04999 67.342048) (width 0.501) (layer F.Cu) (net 2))
 (segment (start 24.04999 67.342048) (end 24.04999 50.49001) (width 0.501) (layer F.Cu) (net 2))
 (segment (start 24.04999 50.49001) (end 24.79 49.75) (width 0.501) (layer F.Cu) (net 2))
 (segment (start 24.79 49.75) (end 26.99 49.75) (width 0.501) (layer F.Cu) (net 2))
 (segment (start 30.92 77) (end 30.920001 79.016001) (width 0.501) (layer F.Cu) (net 3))
 (segment (start 30.920001 79.016001) (end 37.663601 79.016001) (width 0.501) (layer F.Cu) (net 3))
 (segment (start 37.663601 79.016001) (end 37.863601 78.816001) (width 0.501) (layer F.Cu) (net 3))
 (segment (start 37.863601 78.816001) (end 37.863601 74.726267) (width 0.501) (layer F.Cu) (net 3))
 (segment (start 37.863601 74.726267) (end 30 66.862666) (width 0.501) (layer F.Cu) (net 3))
 (segment (start 30 66.862666) (end 30 66) (width 0.501) (layer F.Cu) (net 3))
 (segment (start 30 66) (end 30 62) (width 0.501) (layer F.Cu) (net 3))
 (segment (start 26 29) (end 20.84999 34.15001) (width 0.501) (layer F.Cu) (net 4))
 (segment (start 20.84999 34.15001) (end 20.84999 67.45399) (width 0.501) (layer F.Cu) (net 4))
 (segment (start 20.84999 67.45399) (end 28.38 74.984) (width 0.501) (layer F.Cu) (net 4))
 (segment (start 28.38 74.984) (end 28.38 77) (width 0.501) (layer F.Cu) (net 4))
 (segment (start 28 27) (end 32.92 27) (width 0.501) (layer F.Cu) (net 4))
 (segment (start 26 29) (end 28 27) (width 0.501) (layer F.Cu) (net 4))
 (via (at 26 29) (size 1.5) (drill 0.8) (layers F.Cu B.Cu) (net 4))
 (segment (start 26 34) (end 26 29) (width 1) (layer B.Cu) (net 4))
 (segment (start 26 35.21) (end 26 34) (width 0.501) (layer F.Cu) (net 4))
 (via (at 26 34) (size 1.5) (drill 0.8) (layers F.Cu B.Cu) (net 4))
 (segment (start 26.99 37.75) (end 26.99 36.2) (width 0.501) (layer F.Cu) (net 4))
 (segment (start 26.99 36.2) (end 26 35.21) (width 0.501) (layer F.Cu) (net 4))
 (segment (start 28.38 77) (end 28.38 78.597332) (width 0.501) (layer F.Cu) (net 4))
 (segment (start 28.38 78.597332) (end 30.298677 80.516011) (width 0.501) (layer F.Cu) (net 4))
 (segment (start 30.298677 80.516011) (end 39.059989 80.516011) (width 0.501) (layer F.Cu) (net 4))
 (segment (start 39.059989 80.516011) (end 42.46 77.116) (width 0.501) (layer F.Cu) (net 4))
 (segment (start 42.46 77.116) (end 42.46 77) (width 0.501) (layer F.Cu) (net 4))
 (segment (start 41.44832 72) (end 38 72) (width 0.501) (layer F.Cu) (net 4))
 (segment (start 38 72) (end 37 71) (width 0.501) (layer F.Cu) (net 4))
 (segment (start 42.46 77) (end 42.46 73.01168) (width 0.501) (layer F.Cu) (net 4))
 (segment (start 42.46 73.01168) (end 41.44832 72) (width 0.501) (layer F.Cu) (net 4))
 (segment (start 24 37.65) (end 26.89 37.65) (width 0.501) (layer F.Cu) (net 4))
 (segment (start 26.89 37.65) (end 26.99 37.75) (width 0.501) (layer F.Cu) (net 4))
 (segment (start 32.7 66) (end 32.7 62.3) (width 0.501) (layer F.Cu) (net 6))
 (segment (start 32.7 62.3) (end 33 62) (width 0.501) (layer F.Cu) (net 6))
 (segment (start 37 66) (end 32.7 66) (width 0.501) (layer F.Cu) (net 6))
 (segment (start 37 66) (end 42.82552 66) (width 0.501) (layer F.Cu) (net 6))
 (segment (start 42.82552 66) (end 43.72416 65.10136) (width 0.501) (layer F.Cu) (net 6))
 (segment (start 49 57.35) (end 49 41.56) (width 0.501) (layer F.Cu) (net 6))
 (segment (start 49 41.56) (end 45.19 37.75) (width 0.501) (layer F.Cu) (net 6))
 (segment (start 45.19 37.75) (end 42.99 37.75) (width 0.501) (layer F.Cu) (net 6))
 (segment (start 47 57.7) (end 48.650001 57.699999) (width 0.501) (layer F.Cu) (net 6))
 (segment (start 48.650001 57.699999) (end 49 57.35) (width 0.501) (layer F.Cu) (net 6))
 (segment (start 43.72416 65.10136) (end 43.72416 60.97584) (width 0.501) (layer F.Cu) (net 6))
 (segment (start 43.72416 60.97584) (end 47 57.7) (width 0.501) (layer F.Cu) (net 6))
 (segment (start 38 33) (end 39.842045 33) (width 0.501) (layer F.Cu) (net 6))
 (segment (start 39.842045 33) (end 42.99 36.147955) (width 0.501) (layer F.Cu) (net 6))
 (segment (start 42.99 36.147955) (end 42.99 36.2) (width 0.501) (layer F.Cu) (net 6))
 (segment (start 42.99 36.2) (end 42.99 37.75) (width 0.501) (layer F.Cu) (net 6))
 (segment (start 38 30) (end 38 27) (width 0.501) (layer F.Cu) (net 6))
 (segment (start 38 33) (end 38 30) (width 0.501) (layer F.Cu) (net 6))
 (segment (start 47 55) (end 47 51.7) (width 0.501) (layer F.Cu) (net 7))
 (segment (start 42.99 51.75) (end 46.95 51.75) (width 0.501) (layer F.Cu) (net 7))
 (segment (start 46.95 51.75) (end 47 51.7) (width 0.501) (layer F.Cu) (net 7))
 (segment (start 47 49) (end 47 47.25) (width 0.501) (layer F.Cu) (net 8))
 (segment (start 47 47.25) (end 45.5 45.75) (width 0.501) (layer F.Cu) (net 8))
 (segment (start 45.5 45.75) (end 45.19 45.75) (width 0.501) (layer F.Cu) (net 8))
 (segment (start 45.19 45.75) (end 42.99 45.75) (width 0.501) (layer F.Cu) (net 8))
 (segment (start 35.7 62) (end 35.8 62) (width 0.501) (layer F.Cu) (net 9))
 (segment (start 35.8 62) (end 40.78999 57.01001) (width 0.501) (layer F.Cu) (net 9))
 (segment (start 40.78999 47.75001) (end 40.79 47.75) (width 0.501) (layer F.Cu) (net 9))
 (segment (start 40.78999 57.01001) (end 40.78999 47.75001) (width 0.501) (layer F.Cu) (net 9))
 (segment (start 40.79 47.75) (end 42.99 47.75) (width 0.501) (layer F.Cu) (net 9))
 (segment (start 24 40.35) (end 24.6 39.75) (width 0.501) (layer F.Cu) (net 10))
 (segment (start 24.6 39.75) (end 26.99 39.75) (width 0.501) (layer F.Cu) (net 10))
 (segment (start 27.3 62) (end 27.3 60.35) (width 0.501) (layer F.Cu) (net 11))
 (segment (start 27.3 60.35) (end 29.19001 58.45999) (width 0.501) (layer F.Cu) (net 11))
 (segment (start 29.19001 58.45999) (end 29.19001 43.75001) (width 0.501) (layer F.Cu) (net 11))
 (segment (start 29.19001 43.75001) (end 29.19 43.75) (width 0.501) (layer F.Cu) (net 11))
 (segment (start 29.19 43.75) (end 26.99 43.75) (width 0.501) (layer F.Cu) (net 11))
 (segment (start 35.3 33) (end 27.590002 33) (width 0.501) (layer F.Cu) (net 12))
 (segment (start 27.590002 33) (end 26.840001 32.249999) (width 0.501) (layer F.Cu) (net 12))
 (segment (start 26.840001 32.249999) (end 25.159999 32.249999) (width 0.501) (layer F.Cu) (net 12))
 (segment (start 25.159999 32.249999) (end 22.349999 35.059999) (width 0.501) (layer F.Cu) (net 12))
 (segment (start 22.349999 35.059999) (end 22.349999 41.900001) (width 0.501) (layer F.Cu) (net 12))
 (segment (start 22.349999 41.900001) (end 22.549999 42.100001) (width 0.501) (layer F.Cu) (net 12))
 (segment (start 22.549999 42.100001) (end 26.639999 42.100001) (width 0.501) (layer F.Cu) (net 12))
 (segment (start 26.639999 42.100001) (end 26.99 41.75) (width 0.501) (layer F.Cu) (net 12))
 (segment (start 35.3 33) (end 35.3 30) (width 0.501) (layer F.Cu) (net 12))
 (segment (start 35.3 30) (end 35.3 27.16) (width 0.501) (layer F.Cu) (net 12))
 (segment (start 35.3 27.16) (end 35.46 27) (width 0.501) (layer F.Cu) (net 12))
 (segment (start 45 77) (end 45 73) (width 0.501) (layer F.Cu) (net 5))
 (segment (start 45 73) (end 46 72) (width 0.501) (layer F.Cu) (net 5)))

